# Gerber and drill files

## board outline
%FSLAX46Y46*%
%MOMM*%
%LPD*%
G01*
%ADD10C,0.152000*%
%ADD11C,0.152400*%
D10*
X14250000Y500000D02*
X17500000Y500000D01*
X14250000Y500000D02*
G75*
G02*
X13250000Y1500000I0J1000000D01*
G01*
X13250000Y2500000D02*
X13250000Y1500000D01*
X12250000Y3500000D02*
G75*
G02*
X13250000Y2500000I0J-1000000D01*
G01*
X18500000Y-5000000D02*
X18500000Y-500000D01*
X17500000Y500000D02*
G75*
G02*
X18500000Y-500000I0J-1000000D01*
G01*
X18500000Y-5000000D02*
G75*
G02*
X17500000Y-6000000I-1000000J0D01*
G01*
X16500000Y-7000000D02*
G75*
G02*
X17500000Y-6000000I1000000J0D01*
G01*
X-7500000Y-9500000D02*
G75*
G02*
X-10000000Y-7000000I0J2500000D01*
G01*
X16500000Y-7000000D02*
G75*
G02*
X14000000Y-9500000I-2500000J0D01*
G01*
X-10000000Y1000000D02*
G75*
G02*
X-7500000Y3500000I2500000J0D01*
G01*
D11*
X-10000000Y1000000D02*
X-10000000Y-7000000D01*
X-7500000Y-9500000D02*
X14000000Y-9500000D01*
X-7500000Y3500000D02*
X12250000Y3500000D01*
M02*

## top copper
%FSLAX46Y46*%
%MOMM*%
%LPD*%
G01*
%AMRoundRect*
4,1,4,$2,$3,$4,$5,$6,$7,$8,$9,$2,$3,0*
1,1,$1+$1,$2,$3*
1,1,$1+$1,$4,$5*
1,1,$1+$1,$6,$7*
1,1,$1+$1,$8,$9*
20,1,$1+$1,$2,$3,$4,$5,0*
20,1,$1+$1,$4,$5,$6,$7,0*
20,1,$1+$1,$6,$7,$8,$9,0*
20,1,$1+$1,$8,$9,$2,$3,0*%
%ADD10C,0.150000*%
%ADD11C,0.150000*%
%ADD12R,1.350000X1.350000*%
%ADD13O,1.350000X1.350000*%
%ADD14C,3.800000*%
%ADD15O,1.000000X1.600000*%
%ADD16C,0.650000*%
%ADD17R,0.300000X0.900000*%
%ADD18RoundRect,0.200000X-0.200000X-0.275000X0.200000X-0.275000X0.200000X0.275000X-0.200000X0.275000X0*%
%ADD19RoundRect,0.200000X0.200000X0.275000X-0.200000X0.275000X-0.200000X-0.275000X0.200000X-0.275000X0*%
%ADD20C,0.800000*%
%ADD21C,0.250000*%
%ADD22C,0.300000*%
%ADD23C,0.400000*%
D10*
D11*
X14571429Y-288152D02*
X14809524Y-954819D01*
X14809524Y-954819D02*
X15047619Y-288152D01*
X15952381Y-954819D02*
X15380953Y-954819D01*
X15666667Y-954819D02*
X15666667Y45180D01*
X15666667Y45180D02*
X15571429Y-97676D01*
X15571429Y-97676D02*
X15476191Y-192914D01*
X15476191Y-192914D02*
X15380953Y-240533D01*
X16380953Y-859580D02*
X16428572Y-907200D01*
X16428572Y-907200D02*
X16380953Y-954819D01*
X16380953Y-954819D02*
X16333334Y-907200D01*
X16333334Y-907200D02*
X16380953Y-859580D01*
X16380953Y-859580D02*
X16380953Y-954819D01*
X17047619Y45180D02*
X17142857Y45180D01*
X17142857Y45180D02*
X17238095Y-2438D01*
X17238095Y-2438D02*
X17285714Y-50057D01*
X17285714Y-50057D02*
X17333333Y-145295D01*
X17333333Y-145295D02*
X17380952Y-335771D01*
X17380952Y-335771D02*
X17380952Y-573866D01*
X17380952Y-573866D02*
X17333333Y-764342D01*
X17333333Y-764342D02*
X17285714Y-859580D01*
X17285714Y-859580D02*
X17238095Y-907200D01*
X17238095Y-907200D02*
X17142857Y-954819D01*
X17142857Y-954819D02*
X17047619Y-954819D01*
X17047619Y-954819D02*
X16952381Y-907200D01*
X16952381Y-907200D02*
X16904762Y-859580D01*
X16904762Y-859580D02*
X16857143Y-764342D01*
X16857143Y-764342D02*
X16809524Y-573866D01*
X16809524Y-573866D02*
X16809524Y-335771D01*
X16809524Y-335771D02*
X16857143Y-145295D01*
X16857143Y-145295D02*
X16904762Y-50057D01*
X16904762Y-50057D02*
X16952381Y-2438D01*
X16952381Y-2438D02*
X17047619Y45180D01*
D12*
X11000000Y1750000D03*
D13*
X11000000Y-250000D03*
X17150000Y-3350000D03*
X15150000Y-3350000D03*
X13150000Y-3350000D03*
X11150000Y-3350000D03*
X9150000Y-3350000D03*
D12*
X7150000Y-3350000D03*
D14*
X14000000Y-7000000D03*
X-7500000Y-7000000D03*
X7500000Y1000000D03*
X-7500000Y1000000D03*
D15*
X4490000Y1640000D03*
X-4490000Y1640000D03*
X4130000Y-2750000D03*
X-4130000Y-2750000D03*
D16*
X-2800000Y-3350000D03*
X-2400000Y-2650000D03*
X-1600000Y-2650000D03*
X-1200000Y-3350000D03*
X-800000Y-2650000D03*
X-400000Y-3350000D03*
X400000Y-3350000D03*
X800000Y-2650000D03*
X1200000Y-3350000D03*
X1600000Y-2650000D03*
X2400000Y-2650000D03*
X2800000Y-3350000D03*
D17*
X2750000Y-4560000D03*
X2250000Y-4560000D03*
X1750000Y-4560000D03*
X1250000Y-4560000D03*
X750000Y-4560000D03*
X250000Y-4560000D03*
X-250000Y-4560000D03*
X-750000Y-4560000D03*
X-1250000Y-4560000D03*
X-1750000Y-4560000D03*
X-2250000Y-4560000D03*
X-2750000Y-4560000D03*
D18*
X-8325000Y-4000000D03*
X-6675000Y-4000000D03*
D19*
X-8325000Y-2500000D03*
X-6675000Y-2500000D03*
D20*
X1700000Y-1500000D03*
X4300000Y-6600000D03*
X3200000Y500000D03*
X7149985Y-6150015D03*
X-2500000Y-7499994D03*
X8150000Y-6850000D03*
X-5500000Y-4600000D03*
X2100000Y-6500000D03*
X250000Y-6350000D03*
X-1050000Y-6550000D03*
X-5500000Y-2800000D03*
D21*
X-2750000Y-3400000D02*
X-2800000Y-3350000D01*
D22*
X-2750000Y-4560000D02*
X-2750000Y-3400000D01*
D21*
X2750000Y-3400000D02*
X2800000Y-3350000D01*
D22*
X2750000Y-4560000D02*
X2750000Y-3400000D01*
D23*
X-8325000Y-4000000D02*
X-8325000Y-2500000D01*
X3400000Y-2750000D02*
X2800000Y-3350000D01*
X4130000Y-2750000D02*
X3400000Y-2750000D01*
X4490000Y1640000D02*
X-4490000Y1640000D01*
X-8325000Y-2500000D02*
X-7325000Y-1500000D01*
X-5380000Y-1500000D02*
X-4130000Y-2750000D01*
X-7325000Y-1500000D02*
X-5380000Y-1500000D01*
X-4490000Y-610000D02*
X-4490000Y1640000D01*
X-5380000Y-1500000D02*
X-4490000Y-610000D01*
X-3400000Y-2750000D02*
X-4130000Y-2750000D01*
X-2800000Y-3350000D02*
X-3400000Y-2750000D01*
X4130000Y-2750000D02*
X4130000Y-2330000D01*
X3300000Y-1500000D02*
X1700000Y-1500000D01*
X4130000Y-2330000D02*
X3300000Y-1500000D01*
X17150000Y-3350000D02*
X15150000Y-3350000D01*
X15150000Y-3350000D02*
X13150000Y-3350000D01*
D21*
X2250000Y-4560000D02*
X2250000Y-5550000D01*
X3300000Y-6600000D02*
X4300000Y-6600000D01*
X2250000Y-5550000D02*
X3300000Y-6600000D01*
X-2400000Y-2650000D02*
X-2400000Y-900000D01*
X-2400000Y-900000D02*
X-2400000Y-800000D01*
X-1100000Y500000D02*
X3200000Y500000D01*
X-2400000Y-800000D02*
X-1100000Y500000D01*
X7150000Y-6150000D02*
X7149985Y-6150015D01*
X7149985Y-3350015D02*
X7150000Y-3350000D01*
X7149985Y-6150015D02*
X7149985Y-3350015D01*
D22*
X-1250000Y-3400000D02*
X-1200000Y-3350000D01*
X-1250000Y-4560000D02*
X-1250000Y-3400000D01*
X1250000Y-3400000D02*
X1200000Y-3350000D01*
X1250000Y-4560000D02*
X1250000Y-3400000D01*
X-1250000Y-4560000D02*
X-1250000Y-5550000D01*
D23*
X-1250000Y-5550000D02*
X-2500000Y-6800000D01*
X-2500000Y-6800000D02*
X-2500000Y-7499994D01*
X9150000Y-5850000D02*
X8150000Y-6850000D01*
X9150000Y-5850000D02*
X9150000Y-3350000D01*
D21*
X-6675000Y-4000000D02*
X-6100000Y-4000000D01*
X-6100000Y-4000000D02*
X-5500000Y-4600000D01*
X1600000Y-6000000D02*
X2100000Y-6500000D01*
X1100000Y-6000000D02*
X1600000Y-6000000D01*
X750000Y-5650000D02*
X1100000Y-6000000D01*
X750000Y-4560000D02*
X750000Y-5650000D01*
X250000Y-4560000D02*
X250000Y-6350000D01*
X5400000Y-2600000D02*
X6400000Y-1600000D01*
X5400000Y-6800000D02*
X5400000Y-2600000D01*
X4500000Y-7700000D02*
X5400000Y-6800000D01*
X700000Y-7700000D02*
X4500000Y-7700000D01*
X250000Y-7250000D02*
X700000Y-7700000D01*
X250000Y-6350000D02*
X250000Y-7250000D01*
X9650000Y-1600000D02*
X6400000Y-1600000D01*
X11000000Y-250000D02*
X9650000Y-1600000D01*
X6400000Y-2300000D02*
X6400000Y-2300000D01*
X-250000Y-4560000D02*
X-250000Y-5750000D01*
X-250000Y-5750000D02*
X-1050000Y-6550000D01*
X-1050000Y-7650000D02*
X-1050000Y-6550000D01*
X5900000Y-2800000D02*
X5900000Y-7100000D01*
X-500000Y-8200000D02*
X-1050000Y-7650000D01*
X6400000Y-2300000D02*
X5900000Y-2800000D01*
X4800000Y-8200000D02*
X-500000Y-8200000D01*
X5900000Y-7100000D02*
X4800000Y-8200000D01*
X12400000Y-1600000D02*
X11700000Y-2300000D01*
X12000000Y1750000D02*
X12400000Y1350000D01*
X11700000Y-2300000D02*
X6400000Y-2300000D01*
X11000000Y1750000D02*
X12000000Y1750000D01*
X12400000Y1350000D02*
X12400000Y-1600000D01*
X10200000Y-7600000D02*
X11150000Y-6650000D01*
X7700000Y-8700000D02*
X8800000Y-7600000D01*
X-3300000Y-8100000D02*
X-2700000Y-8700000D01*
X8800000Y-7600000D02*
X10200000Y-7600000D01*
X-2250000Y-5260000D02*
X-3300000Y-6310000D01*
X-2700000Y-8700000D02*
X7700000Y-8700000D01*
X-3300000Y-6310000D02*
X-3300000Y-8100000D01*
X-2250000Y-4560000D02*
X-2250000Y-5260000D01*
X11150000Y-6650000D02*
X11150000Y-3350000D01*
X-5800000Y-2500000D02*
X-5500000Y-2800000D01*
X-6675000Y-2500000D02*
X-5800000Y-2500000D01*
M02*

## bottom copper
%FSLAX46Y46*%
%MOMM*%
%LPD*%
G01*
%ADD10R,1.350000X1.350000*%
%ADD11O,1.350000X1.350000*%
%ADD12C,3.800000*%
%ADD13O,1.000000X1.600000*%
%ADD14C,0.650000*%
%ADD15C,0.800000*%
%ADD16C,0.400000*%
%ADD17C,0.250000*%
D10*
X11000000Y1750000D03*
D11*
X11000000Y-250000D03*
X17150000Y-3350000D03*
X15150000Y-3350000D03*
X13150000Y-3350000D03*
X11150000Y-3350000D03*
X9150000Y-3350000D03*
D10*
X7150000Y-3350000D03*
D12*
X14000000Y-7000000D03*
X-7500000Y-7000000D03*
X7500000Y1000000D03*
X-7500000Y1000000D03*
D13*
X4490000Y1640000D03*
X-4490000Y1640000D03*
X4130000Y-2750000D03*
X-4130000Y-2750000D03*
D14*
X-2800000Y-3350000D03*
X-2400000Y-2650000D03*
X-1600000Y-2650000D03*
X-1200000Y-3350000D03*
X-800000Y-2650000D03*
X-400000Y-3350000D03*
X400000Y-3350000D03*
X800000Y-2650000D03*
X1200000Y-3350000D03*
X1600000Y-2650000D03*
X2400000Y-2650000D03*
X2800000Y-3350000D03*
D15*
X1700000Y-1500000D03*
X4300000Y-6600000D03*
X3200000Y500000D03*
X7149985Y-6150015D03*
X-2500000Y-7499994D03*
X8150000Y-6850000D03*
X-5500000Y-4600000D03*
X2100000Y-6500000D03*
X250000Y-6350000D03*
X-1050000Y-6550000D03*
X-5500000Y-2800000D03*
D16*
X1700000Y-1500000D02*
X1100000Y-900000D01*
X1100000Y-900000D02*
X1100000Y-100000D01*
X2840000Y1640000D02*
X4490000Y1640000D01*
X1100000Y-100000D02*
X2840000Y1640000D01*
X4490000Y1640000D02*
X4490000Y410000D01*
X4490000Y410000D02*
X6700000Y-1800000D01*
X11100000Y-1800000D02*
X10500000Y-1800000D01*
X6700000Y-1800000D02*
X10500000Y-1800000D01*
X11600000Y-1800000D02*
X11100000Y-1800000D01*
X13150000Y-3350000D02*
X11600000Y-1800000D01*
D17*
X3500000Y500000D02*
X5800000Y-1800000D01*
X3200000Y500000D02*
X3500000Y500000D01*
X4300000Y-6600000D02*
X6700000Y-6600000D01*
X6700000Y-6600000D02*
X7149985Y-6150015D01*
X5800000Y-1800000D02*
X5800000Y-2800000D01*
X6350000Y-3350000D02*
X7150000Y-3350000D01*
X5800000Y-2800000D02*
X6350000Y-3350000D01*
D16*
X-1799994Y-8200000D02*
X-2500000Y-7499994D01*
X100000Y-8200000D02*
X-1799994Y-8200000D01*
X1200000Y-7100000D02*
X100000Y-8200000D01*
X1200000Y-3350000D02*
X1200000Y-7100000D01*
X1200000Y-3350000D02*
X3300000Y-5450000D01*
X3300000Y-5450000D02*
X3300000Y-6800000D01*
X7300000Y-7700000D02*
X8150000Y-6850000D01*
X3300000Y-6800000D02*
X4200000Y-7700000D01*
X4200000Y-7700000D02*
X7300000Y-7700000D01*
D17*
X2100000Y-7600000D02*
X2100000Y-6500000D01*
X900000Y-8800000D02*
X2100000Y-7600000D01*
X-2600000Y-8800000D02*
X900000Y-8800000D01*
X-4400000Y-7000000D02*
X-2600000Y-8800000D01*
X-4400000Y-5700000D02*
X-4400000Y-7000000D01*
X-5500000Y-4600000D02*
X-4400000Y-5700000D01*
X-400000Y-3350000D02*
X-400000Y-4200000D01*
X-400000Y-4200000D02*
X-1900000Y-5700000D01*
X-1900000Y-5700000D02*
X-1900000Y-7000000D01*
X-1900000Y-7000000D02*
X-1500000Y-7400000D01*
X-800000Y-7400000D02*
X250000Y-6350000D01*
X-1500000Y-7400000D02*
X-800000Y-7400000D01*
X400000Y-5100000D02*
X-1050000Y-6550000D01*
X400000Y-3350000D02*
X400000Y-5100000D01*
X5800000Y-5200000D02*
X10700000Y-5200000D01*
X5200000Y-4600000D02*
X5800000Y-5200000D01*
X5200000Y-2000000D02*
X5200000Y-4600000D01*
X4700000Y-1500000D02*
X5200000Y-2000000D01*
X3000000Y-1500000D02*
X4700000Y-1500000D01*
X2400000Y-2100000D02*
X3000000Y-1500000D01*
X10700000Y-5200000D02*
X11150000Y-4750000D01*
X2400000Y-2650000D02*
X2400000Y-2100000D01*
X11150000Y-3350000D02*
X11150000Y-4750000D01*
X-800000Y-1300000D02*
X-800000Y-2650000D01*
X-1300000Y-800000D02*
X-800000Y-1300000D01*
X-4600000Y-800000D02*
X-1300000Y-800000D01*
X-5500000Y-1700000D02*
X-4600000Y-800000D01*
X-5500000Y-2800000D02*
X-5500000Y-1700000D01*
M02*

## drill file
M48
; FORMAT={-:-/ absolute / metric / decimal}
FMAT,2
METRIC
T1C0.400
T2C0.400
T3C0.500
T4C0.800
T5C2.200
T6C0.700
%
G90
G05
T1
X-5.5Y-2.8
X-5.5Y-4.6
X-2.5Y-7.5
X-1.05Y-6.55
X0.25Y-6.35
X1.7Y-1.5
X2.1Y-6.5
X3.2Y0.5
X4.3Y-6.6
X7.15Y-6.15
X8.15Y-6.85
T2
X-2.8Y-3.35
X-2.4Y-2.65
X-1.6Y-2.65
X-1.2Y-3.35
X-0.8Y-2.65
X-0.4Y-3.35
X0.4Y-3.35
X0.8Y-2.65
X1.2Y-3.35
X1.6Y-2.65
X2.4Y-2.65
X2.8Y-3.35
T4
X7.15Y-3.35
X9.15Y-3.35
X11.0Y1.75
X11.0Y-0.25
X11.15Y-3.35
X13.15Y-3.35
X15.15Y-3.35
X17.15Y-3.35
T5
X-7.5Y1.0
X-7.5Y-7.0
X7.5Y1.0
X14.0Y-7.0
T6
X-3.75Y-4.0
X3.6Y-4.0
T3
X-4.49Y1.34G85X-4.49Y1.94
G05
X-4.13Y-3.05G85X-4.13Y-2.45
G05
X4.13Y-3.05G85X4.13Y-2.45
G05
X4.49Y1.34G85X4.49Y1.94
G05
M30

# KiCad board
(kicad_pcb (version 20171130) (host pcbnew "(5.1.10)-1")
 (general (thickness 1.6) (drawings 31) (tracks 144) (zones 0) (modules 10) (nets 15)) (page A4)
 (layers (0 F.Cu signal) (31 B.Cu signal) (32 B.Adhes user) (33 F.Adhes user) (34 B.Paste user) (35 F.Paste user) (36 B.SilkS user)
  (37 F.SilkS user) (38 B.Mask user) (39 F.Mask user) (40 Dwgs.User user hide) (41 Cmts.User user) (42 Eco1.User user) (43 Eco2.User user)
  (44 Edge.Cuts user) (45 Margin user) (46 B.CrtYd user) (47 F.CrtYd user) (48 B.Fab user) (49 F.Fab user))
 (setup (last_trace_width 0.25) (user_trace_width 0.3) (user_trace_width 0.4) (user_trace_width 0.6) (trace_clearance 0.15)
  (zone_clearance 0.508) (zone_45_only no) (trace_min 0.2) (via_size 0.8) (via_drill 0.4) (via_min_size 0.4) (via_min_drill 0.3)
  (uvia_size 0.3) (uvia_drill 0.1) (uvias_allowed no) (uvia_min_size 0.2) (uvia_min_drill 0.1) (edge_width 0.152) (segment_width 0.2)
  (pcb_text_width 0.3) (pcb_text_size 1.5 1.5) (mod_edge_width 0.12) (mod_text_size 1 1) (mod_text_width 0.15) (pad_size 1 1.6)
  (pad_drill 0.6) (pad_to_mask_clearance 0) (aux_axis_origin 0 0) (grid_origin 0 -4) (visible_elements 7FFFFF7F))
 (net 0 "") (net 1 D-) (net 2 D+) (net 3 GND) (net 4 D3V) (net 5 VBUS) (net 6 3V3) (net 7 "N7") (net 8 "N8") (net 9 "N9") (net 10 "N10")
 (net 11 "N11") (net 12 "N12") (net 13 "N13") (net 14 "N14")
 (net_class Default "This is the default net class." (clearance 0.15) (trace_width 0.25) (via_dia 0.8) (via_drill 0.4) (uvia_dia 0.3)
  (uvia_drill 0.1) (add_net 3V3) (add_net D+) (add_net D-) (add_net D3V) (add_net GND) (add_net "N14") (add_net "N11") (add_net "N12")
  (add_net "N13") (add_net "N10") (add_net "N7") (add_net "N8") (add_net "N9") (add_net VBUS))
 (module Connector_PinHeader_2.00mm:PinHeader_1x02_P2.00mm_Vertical (layer F.Cu) (at 11 -1.75)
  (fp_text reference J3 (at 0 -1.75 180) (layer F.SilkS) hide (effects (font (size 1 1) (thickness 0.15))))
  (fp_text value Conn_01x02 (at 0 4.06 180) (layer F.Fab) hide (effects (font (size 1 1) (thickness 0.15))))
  (pad 1 thru_hole rect (at 0 0) (size 1.35 1.35) (drill 0.8) (layers *.Cu *.Mask) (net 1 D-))
  (pad 2 thru_hole oval (at 0 2) (size 1.35 1.35) (drill 0.8) (layers *.Cu *.Mask) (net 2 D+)))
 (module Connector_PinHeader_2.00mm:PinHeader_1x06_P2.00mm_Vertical (layer F.Cu) (at 7.15 3.35 90)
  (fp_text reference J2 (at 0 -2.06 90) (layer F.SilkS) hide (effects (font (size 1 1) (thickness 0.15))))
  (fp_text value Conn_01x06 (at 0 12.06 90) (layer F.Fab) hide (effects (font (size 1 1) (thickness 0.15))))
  (pad 6 thru_hole oval (at 0 10 90) (size 1.35 1.35) (drill 0.8) (layers *.Cu *.Mask) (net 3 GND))
  (pad 5 thru_hole oval (at 0 8 90) (size 1.35 1.35) (drill 0.8) (layers *.Cu *.Mask) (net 3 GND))
  (pad 4 thru_hole oval (at 0 6 90) (size 1.35 1.35) (drill 0.8) (layers *.Cu *.Mask) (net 3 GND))
  (pad 3 thru_hole oval (at 0 4 90) (size 1.35 1.35) (drill 0.8) (layers *.Cu *.Mask) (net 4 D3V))
  (pad 2 thru_hole oval (at 0 2 90) (size 1.35 1.35) (drill 0.8) (layers *.Cu *.Mask) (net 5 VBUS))
  (pad 1 thru_hole rect (at 0 0 90) (size 1.35 1.35) (drill 0.8) (layers *.Cu *.Mask) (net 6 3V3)))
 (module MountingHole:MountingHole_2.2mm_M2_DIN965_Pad (layer F.Cu) (at 14 7)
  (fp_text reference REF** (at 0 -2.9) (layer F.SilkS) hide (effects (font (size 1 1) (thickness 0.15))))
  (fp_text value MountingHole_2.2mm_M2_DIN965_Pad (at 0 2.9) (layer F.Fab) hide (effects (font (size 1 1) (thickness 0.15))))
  (pad 1 thru_hole circle (at 0 0) (size 3.8 3.8) (drill 2.2) (layers *.Cu *.Mask)))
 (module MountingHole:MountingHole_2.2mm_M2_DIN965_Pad (layer F.Cu) (at -7.5 7)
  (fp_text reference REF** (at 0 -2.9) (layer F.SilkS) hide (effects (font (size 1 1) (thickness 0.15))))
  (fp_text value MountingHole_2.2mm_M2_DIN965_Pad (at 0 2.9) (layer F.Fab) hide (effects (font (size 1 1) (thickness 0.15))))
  (pad 1 thru_hole circle (at 0 0) (size 3.8 3.8) (drill 2.2) (layers *.Cu *.Mask)))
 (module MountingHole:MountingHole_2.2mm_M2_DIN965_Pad (layer F.Cu) (at 7.5 -1)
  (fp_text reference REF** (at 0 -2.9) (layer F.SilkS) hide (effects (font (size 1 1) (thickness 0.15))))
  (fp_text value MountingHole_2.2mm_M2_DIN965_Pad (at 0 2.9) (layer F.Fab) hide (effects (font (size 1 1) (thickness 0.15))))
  (pad 1 thru_hole circle (at 0 0) (size 3.8 3.8) (drill 2.2) (layers *.Cu *.Mask)))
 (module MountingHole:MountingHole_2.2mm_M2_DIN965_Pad (layer F.Cu) (at -7.5 -1)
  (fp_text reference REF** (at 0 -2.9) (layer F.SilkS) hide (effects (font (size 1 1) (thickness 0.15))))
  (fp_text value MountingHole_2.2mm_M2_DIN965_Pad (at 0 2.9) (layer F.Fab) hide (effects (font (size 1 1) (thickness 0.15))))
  (pad 1 thru_hole circle (at 0 0) (size 3.8 3.8) (drill 2.2) (layers *.Cu *.Mask)))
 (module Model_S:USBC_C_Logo (layer F.Cu) (at -3.5 7.5)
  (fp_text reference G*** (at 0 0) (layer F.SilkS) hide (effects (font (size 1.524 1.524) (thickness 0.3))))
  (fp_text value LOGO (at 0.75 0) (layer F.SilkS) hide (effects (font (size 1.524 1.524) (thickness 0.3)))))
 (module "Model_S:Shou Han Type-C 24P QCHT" (layer F.Cu) (at 0 -3.5 180)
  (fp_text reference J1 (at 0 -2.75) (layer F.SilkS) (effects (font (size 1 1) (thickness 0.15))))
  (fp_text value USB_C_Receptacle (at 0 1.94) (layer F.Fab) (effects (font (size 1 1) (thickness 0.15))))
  (pad S1 thru_hole oval (at -4.49 -1.86 180) (size 1 1.6) (drill oval 0.5 1.1) (layers *.Cu *.Mask) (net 3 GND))
  (pad S1 thru_hole oval (at 4.49 -1.86 180) (size 1 1.6) (drill oval 0.5 1.1) (layers *.Cu *.Mask) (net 3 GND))
  (pad S1 thru_hole oval (at -4.13 -6.25 180) (size 1 1.6) (drill oval 0.5 1.1) (layers *.Cu *.Mask) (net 3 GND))
  (pad S1 thru_hole oval (at 4.13 -6.25 180) (size 1 1.6) (drill oval 0.5 1.1) (layers *.Cu *.Mask) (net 3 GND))
  (pad B1 thru_hole circle (at 2.8 -6.85 180) (size 0.65 0.65) (drill 0.4) (layers *.Cu *.Mask) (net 3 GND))
  (pad B2 thru_hole circle (at 2.4 -6.15 180) (size 0.65 0.65) (drill 0.4) (layers *.Cu *.Mask) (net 6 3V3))
  (pad B3 thru_hole circle (at 1.6 -6.15 180) (size 0.65 0.65) (drill 0.4) (layers *.Cu *.Mask) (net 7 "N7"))
  (pad B4 thru_hole circle (at 1.2 -6.85 180) (size 0.65 0.65) (drill 0.4) (layers *.Cu *.Mask) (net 5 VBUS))
  (pad B5 thru_hole circle (at 0.8 -6.15 180) (size 0.65 0.65) (drill 0.4) (layers *.Cu *.Mask) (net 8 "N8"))
  (pad B6 thru_hole circle (at 0.4 -6.85 180) (size 0.65 0.65) (drill 0.4) (layers *.Cu *.Mask) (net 2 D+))
  (pad B7 thru_hole circle (at -0.4 -6.85 180) (size 0.65 0.65) (drill 0.4) (layers *.Cu *.Mask) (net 1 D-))
  (pad B8 thru_hole circle (at -0.8 -6.15 180) (size 0.65 0.65) (drill 0.4) (layers *.Cu *.Mask) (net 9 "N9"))
  (pad B9 thru_hole circle (at -1.2 -6.85 180) (size 0.65 0.65) (drill 0.4) (layers *.Cu *.Mask) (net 5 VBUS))
  (pad B10 thru_hole circle (at -1.6 -6.15 180) (size 0.65 0.65) (drill 0.4) (layers *.Cu *.Mask) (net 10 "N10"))
  (pad B11 thru_hole circle (at -2.4 -6.15 180) (size 0.65 0.65) (drill 0.4) (layers *.Cu *.Mask) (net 4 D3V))
  (pad B12 thru_hole circle (at -2.8 -6.85 180) (size 0.65 0.65) (drill 0.4) (layers *.Cu *.Mask) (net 3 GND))
  (pad "" np_thru_hole circle (at -3.6 -7.5 180) (size 0.7 0.7) (drill 0.7) (layers *.Cu *.Mask))
  (pad "" np_thru_hole circle (at 3.75 -7.5 180) (size 0.7 0.7) (drill 0.7) (layers *.Cu *.Mask))
  (pad A1 smd rect (at -2.75 -8.06 180) (size 0.3 0.9) (layers F.Cu F.Paste F.Mask) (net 3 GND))
  (pad A2 smd rect (at -2.25 -8.06 180) (size 0.3 0.9) (layers F.Cu F.Paste F.Mask) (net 6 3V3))
  (pad A3 smd rect (at -1.75 -8.06 180) (size 0.3 0.9) (layers F.Cu F.Paste F.Mask) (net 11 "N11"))
  (pad A4 smd rect (at -1.25 -8.06 180) (size 0.3 0.9) (layers F.Cu F.Paste F.Mask) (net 5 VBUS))
  (pad A5 smd rect (at -0.75 -8.06 180) (size 0.3 0.9) (layers F.Cu F.Paste F.Mask) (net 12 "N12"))
  (pad A6 smd rect (at -0.25 -8.06 180) (size 0.3 0.9) (layers F.Cu F.Paste F.Mask) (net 2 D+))
  (pad A7 smd rect (at 0.25 -8.06 180) (size 0.3 0.9) (layers F.Cu F.Paste F.Mask) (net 1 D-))
  (pad A8 smd rect (at 0.75 -8.06 180) (size 0.3 0.9) (layers F.Cu F.Paste F.Mask) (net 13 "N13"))
  (pad A9 smd rect (at 1.25 -8.06 180) (size 0.3 0.9) (layers F.Cu F.Paste F.Mask) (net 5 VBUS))
  (pad A10 smd rect (at 1.75 -8.06 180) (size 0.3 0.9) (layers F.Cu F.Paste F.Mask) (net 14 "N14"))
  (pad A11 smd rect (at 2.25 -8.06 180) (size 0.3 0.9) (layers F.Cu F.Paste F.Mask) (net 4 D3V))
  (pad A12 smd rect (at 2.75 -8.06 180) (size 0.3 0.9) (layers F.Cu F.Paste F.Mask) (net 3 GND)))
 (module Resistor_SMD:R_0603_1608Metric (layer F.Cu) (at -7.5 4)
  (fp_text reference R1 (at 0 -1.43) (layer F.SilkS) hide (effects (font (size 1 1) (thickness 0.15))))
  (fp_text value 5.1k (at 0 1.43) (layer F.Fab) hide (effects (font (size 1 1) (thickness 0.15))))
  (pad 1 smd roundrect (at -0.825 0) (size 0.8 0.95) (layers F.Cu F.Paste F.Mask) (roundrect_rratio 0.25) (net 3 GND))
  (pad 2 smd roundrect (at 0.825 0) (size 0.8 0.95) (layers F.Cu F.Paste F.Mask) (roundrect_rratio 0.25) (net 12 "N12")))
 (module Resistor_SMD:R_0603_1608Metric (layer F.Cu) (at -7.5 2.5 180)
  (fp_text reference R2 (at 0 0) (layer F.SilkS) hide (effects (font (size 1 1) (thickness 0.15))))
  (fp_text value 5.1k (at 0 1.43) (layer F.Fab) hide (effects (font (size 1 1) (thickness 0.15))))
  (pad 2 smd roundrect (at 0.825 0 180) (size 0.8 0.95) (layers F.Cu F.Paste F.Mask) (roundrect_rratio 0.25) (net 3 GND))
  (pad 1 smd roundrect (at -0.825 0 180) (size 0.8 0.95) (layers F.Cu F.Paste F.Mask) (roundrect_rratio 0.25) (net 8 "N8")))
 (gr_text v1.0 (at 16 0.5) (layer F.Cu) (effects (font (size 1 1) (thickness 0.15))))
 (gr_line (start 14.25 -0.5) (end 17.5 -0.5) (layer Edge.Cuts) (width 0.152))
 (gr_arc (start 14.25 -1.5) (end 13.25 -1.5) (angle -90) (layer Edge.Cuts) (width 0.152))
 (gr_line (start 13.25 -2.5) (end 13.25 -1.5) (layer Edge.Cuts) (width 0.152))
 (gr_arc (start 12.25 -2.5) (end 13.25 -2.5) (angle -90) (layer Edge.Cuts) (width 0.152))
 (gr_line (start 18.5 5) (end 18.5 0.5) (layer Edge.Cuts) (width 0.152))
 (gr_arc (start 17.5 0.5) (end 18.5 0.5) (angle -90) (layer Edge.Cuts) (width 0.152))
 (gr_arc (start 17.5 5) (end 17.5 6) (angle -90) (layer Edge.Cuts) (width 0.152))
 (gr_arc (start 17.5 7) (end 17.5 6) (angle -90) (layer Edge.Cuts) (width 0.152))
 (gr_arc (start -7.5 7) (end -10 7) (angle -90) (layer Edge.Cuts) (width 0.152))
 (gr_arc (start 14 7) (end 14 9.5) (angle -90) (layer Edge.Cuts) (width 0.152))
 (gr_arc (start -7.5 -1) (end -7.5 -3.5) (angle -90) (layer Edge.Cuts) (width 0.152))
 (gr_line (start -10 -1) (end -10 7) (layer Edge.Cuts) (width 0.1524))
 (gr_line (start -7.5 9.5) (end 14 9.5) (layer Edge.Cuts) (width 0.1524))
 (gr_line (start -7.5 -3.5) (end 12.25 -3.5) (layer Edge.Cuts) (width 0.1524))
 (segment (start -2.75 3.4) (end -2.8 3.35) (width 0.25) (layer F.Cu) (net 3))
 (segment (start -2.75 4.56) (end -2.75 3.4) (width 0.3) (layer F.Cu) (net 3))
 (segment (start 2.75 3.4) (end 2.8 3.35) (width 0.25) (layer F.Cu) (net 3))
 (segment (start 2.75 4.56) (end 2.75 3.4) (width 0.3) (layer F.Cu) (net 3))
 (segment (start -8.325 4) (end -8.325 2.5) (width 0.4) (layer F.Cu) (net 3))
 (segment (start 3.4 2.75) (end 2.8 3.35) (width 0.4) (layer F.Cu) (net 3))
 (segment (start 4.13 2.75) (end 3.4 2.75) (width 0.4) (layer F.Cu) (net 3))
 (segment (start 4.49 -1.64) (end -4.49 -1.64) (width 0.4) (layer F.Cu) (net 3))
 (segment (start -8.325 2.5) (end -7.325 1.5) (width 0.4) (layer F.Cu) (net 3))
 (segment (start -5.38 1.5) (end -4.13 2.75) (width 0.4) (layer F.Cu) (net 3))
 (segment (start -7.325 1.5) (end -5.38 1.5) (width 0.4) (layer F.Cu) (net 3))
 (segment (start -4.49 0.61) (end -4.49 -1.64) (width 0.4) (layer F.Cu) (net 3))
 (segment (start -5.38 1.5) (end -4.49 0.61) (width 0.4) (layer F.Cu) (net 3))
 (segment (start -3.4 2.75) (end -4.13 2.75) (width 0.4) (layer F.Cu) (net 3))
 (segment (start -2.8 3.35) (end -3.4 2.75) (width 0.4) (layer F.Cu) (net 3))
 (segment (start 4.13 2.75) (end 4.13 2.33) (width 0.4) (layer F.Cu) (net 3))
 (via (at 1.7 1.5) (size 0.8) (drill 0.4) (layers F.Cu B.Cu) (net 3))
 (segment (start 3.3 1.5) (end 1.7 1.5) (width 0.4) (layer F.Cu) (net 3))
 (segment (start 4.13 2.33) (end 3.3 1.5) (width 0.4) (layer F.Cu) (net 3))
 (segment (start 1.7 1.5) (end 1.1 0.9) (width 0.4) (layer B.Cu) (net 3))
 (segment (start 1.1 0.9) (end 1.1 0.1) (width 0.4) (layer B.Cu) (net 3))
 (segment (start 2.84 -1.64) (end 4.49 -1.64) (width 0.4) (layer B.Cu) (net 3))
 (segment (start 1.1 0.1) (end 2.84 -1.64) (width 0.4) (layer B.Cu) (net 3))
 (segment (start 4.49 -1.64) (end 4.49 -0.41) (width 0.4) (layer B.Cu) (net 3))
 (segment (start 4.49 -0.41) (end 6.7 1.8) (width 0.4) (layer B.Cu) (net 3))
 (segment (start 11.1 1.8) (end 10.5 1.8) (width 0.4) (layer B.Cu) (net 3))
 (segment (start 6.7 1.8) (end 10.5 1.8) (width 0.4) (layer B.Cu) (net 3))
 (segment (start 17.15 3.35) (end 15.15 3.35) (width 0.4) (layer F.Cu) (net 3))
 (segment (start 15.15 3.35) (end 13.15 3.35) (width 0.4) (layer F.Cu) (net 3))
 (segment (start 11.6 1.8) (end 11.1 1.8) (width 0.4) (layer B.Cu) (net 3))
 (segment (start 13.15 3.35) (end 11.6 1.8) (width 0.4) (layer B.Cu) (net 3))
 (segment (start 2.25 4.56) (end 2.25 5.55) (width 0.25) (layer F.Cu) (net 6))
 (via (at 4.3 6.6) (size 0.8) (drill 0.4) (layers F.Cu B.Cu) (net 6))
 (segment (start 3.3 6.6) (end 4.3 6.6) (width 0.25) (layer F.Cu) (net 6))
 (segment (start 2.25 5.55) (end 3.3 6.6) (width 0.25) (layer F.Cu) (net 6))
 (segment (start -2.4 2.65) (end -2.4 0.9) (width 0.25) (layer F.Cu) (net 6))
 (segment (start -2.4 0.9) (end -2.4 0.8) (width 0.25) (layer F.Cu) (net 6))
 (via (at 3.2 -0.5) (size 0.8) (drill 0.4) (layers F.Cu B.Cu) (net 6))
 (segment (start -1.1 -0.5) (end 3.2 -0.5) (width 0.25) (layer F.Cu) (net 6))
 (segment (start -2.4 0.8) (end -1.1 -0.5) (width 0.25) (layer F.Cu) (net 6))
 (segment (start 3.5 -0.5) (end 5.8 1.8) (width 0.25) (layer B.Cu) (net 6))
 (segment (start 3.2 -0.5) (end 3.5 -0.5) (width 0.25) (layer B.Cu) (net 6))
 (segment (start 4.3 6.6) (end 6.7 6.6) (width 0.25) (layer B.Cu) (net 6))
 (via (at 7.149985 6.150015) (size 0.8) (drill 0.4) (layers F.Cu B.Cu) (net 6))
 (segment (start 6.7 6.6) (end 7.149985 6.150015) (width 0.25) (layer B.Cu) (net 6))
 (segment (start 7.15 6.15) (end 7.149985 6.150015) (width 0.25) (layer F.Cu) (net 6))
 (segment (start 7.149985 3.350015) (end 7.15 3.35) (width 0.25) (layer F.Cu) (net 6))
 (segment (start 7.149985 6.150015) (end 7.149985 3.350015) (width 0.25) (layer F.Cu) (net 6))
 (segment (start 5.8 1.8) (end 5.8 2.8) (width 0.25) (layer B.Cu) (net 6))
 (segment (start 6.35 3.35) (end 7.15 3.35) (width 0.25) (layer B.Cu) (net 6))
 (segment (start 5.8 2.8) (end 6.35 3.35) (width 0.25) (layer B.Cu) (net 6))
 (segment (start -1.25 3.4) (end -1.2 3.35) (width 0.3) (layer F.Cu) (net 5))
 (segment (start -1.25 4.56) (end -1.25 3.4) (width 0.3) (layer F.Cu) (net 5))
 (segment (start 1.25 3.4) (end 1.2 3.35) (width 0.3) (layer F.Cu) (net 5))
 (segment (start 1.25 4.56) (end 1.25 3.4) (width 0.3) (layer F.Cu) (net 5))
 (segment (start -1.25 4.56) (end -1.25 5.55) (width 0.3) (layer F.Cu) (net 5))
 (via (at -2.5 7.499994) (size 0.8) (drill 0.4) (layers F.Cu B.Cu) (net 5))
 (segment (start -1.25 5.55) (end -2.5 6.8) (width 0.4) (layer F.Cu) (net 5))
 (segment (start -2.5 6.8) (end -2.5 7.499994) (width 0.4) (layer F.Cu) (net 5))
 (segment (start -1.799994 8.2) (end -2.5 7.499994) (width 0.4) (layer B.Cu) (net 5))
 (segment (start 0.1 8.2) (end -1.799994 8.2) (width 0.4) (layer B.Cu) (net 5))
 (segment (start 1.2 7.1) (end 0.1 8.2) (width 0.4) (layer B.Cu) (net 5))
 (segment (start 1.2 3.35) (end 1.2 7.1) (width 0.4) (layer B.Cu) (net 5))
 (via (at 8.15 6.85) (size 0.8) (drill 0.4) (layers F.Cu B.Cu) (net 5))
 (segment (start 9.15 5.85) (end 8.15 6.85) (width 0.4) (layer F.Cu) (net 5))
 (segment (start 1.2 3.35) (end 3.3 5.45) (width 0.4) (layer B.Cu) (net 5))
 (segment (start 3.3 5.45) (end 3.3 6.8) (width 0.4) (layer B.Cu) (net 5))
 (segment (start 7.3 7.7) (end 8.15 6.85) (width 0.4) (layer B.Cu) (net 5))
 (segment (start 3.3 6.8) (end 4.2 7.7) (width 0.4) (layer B.Cu) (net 5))
 (segment (start 4.2 7.7) (end 7.3 7.7) (width 0.4) (layer B.Cu) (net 5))
 (segment (start 9.15 5.85) (end 9.15 3.35) (width 0.4) (layer F.Cu) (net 5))
 (segment (start -6.675 4) (end -6.1 4) (width 0.25) (layer F.Cu) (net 12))
 (via (at -5.5 4.6) (size 0.8) (drill 0.4) (layers F.Cu B.Cu) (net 12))
 (segment (start -6.1 4) (end -5.5 4.6) (width 0.25) (layer F.Cu) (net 12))
 (via (at 2.1 6.5) (size 0.8) (drill 0.4) (layers F.Cu B.Cu) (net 12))
 (segment (start 1.6 6) (end 2.1 6.5) (width 0.25) (layer F.Cu) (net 12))
 (segment (start 1.1 6) (end 1.6 6) (width 0.25) (layer F.Cu) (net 12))
 (segment (start 0.75 5.65) (end 1.1 6) (width 0.25) (layer F.Cu) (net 12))
 (segment (start 0.75 4.56) (end 0.75 5.65) (width 0.25) (layer F.Cu) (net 12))
 (segment (start 2.1 7.6) (end 2.1 6.5) (width 0.25) (layer B.Cu) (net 12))
 (segment (start 0.9 8.8) (end 2.1 7.6) (width 0.25) (layer B.Cu) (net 12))
 (segment (start -2.6 8.8) (end 0.9 8.8) (width 0.25) (layer B.Cu) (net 12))
 (segment (start -4.4 7) (end -2.6 8.8) (width 0.25) (layer B.Cu) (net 12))
 (segment (start -4.4 5.7) (end -4.4 7) (width 0.25) (layer B.Cu) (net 12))
 (segment (start -5.5 4.6) (end -4.4 5.7) (width 0.25) (layer B.Cu) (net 12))
 (segment (start -0.4 3.35) (end -0.4 4.2) (width 0.25) (layer B.Cu) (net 2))
 (segment (start -0.4 4.2) (end -1.9 5.7) (width 0.25) (layer B.Cu) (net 2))
 (segment (start -1.9 5.7) (end -1.9 7) (width 0.25) (layer B.Cu) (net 2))
 (segment (start -1.9 7) (end -1.5 7.4) (width 0.25) (layer B.Cu) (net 2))
 (via (at 0.25 6.35) (size 0.8) (drill 0.4) (layers F.Cu B.Cu) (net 2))
 (segment (start -0.8 7.4) (end 0.25 6.35) (width 0.25) (layer B.Cu) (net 2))
 (segment (start -1.5 7.4) (end -0.8 7.4) (width 0.25) (layer B.Cu) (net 2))
 (segment (start 0.25 4.56) (end 0.25 6.35) (width 0.25) (layer F.Cu) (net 2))
 (segment (start 5.4 2.6) (end 6.4 1.6) (width 0.25) (layer F.Cu) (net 2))
 (segment (start 5.4 6.8) (end 5.4 2.6) (width 0.25) (layer F.Cu) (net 2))
 (segment (start 4.5 7.7) (end 5.4 6.8) (width 0.25) (layer F.Cu) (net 2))
 (segment (start 0.7 7.7) (end 4.5 7.7) (width 0.25) (layer F.Cu) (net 2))
 (segment (start 0.25 7.25) (end 0.7 7.7) (width 0.25) (layer F.Cu) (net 2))
 (segment (start 0.25 6.35) (end 0.25 7.25) (width 0.25) (layer F.Cu) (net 2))
 (segment (start 9.65 1.6) (end 6.4 1.6) (width 0.25) (layer F.Cu) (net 2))
 (segment (start 11 0.25) (end 9.65 1.6) (width 0.25) (layer F.Cu) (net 2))
 (segment (start 6.4 2.3) (end 6.4 2.3) (width 0.25) (layer F.Cu) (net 1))
 (segment (start 0.4 5.1) (end -1.05 6.55) (width 0.25) (layer B.Cu) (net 1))
 (segment (start 0.4 3.35) (end 0.4 5.1) (width 0.25) (layer B.Cu) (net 1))
 (segment (start -0.25 4.56) (end -0.25 5.75) (width 0.25) (layer F.Cu) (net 1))
 (segment (start -0.25 5.75) (end -1.05 6.55) (width 0.25) (layer F.Cu) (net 1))
 (via (at -1.05 6.55) (size 0.8) (drill 0.4) (layers F.Cu B.Cu) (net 1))
 (segment (start -1.05 7.65) (end -1.05 6.55) (width 0.25) (layer F.Cu) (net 1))
 (segment (start 5.9 2.8) (end 5.9 7.1) (width 0.25) (layer F.Cu) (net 1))
 (segment (start -0.5 8.2) (end -1.05 7.65) (width 0.25) (layer F.Cu) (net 1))
 (segment (start 6.4 2.3) (end 5.9 2.8) (width 0.25) (layer F.Cu) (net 1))
 (segment (start 4.8 8.2) (end -0.5 8.2) (width 0.25) (layer F.Cu) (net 1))
 (segment (start 5.9 7.1) (end 4.8 8.2) (width 0.25) (layer F.Cu) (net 1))
 (segment (start 12.4 1.6) (end 11.7 2.3) (width 0.25) (layer F.Cu) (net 1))
 (segment (start 12 -1.75) (end 12.4 -1.35) (width 0.25) (layer F.Cu) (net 1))
 (segment (start 11.7 2.3) (end 6.4 2.3) (width 0.25) (layer F.Cu) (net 1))
 (segment (start 11 -1.75) (end 12 -1.75) (width 0.25) (layer F.Cu) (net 1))
 (segment (start 12.4 -1.35) (end 12.4 1.6) (width 0.25) (layer F.Cu) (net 1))
 (segment (start 5.8 5.2) (end 10.7 5.2) (width 0.25) (layer B.Cu) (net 4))
 (segment (start 5.2 4.6) (end 5.8 5.2) (width 0.25) (layer B.Cu) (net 4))
 (segment (start 5.2 2) (end 5.2 4.6) (width 0.25) (layer B.Cu) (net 4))
 (segment (start 4.7 1.5) (end 5.2 2) (width 0.25) (layer B.Cu) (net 4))
 (segment (start 3 1.5) (end 4.7 1.5) (width 0.25) (layer B.Cu) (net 4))
 (segment (start 2.4 2.1) (end 3 1.5) (width 0.25) (layer B.Cu) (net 4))
 (segment (start 10.7 5.2) (end 11.15 4.75) (width 0.25) (layer B.Cu) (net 4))
 (segment (start 2.4 2.65) (end 2.4 2.1) (width 0.25) (layer B.Cu) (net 4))
 (segment (start 10.2 7.6) (end 11.15 6.65) (width 0.25) (layer F.Cu) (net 4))
 (segment (start 7.7 8.7) (end 8.8 7.6) (width 0.25) (layer F.Cu) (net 4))
 (segment (start -3.3 8.1) (end -2.7 8.7) (width 0.25) (layer F.Cu) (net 4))
 (segment (start 8.8 7.6) (end 10.2 7.6) (width 0.25) (layer F.Cu) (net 4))
 (segment (start -2.25 5.26) (end -3.3 6.31) (width 0.25) (layer F.Cu) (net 4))
 (segment (start -2.7 8.7) (end 7.7 8.7) (width 0.25) (layer F.Cu) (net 4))
 (segment (start -3.3 6.31) (end -3.3 8.1) (width 0.25) (layer F.Cu) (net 4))
 (segment (start -2.25 4.56) (end -2.25 5.26) (width 0.25) (layer F.Cu) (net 4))
 (segment (start 11.15 3.35) (end 11.15 4.75) (width 0.25) (layer B.Cu) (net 4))
 (segment (start 11.15 6.65) (end 11.15 3.35) (width 0.25) (layer F.Cu) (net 4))
 (via (at -5.5 2.8) (size 0.8) (drill 0.4) (layers F.Cu B.Cu) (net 8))
 (segment (start -5.8 2.5) (end -5.5 2.8) (width 0.25) (layer F.Cu) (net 8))
 (segment (start -6.675 2.5) (end -5.8 2.5) (width 0.25) (layer F.Cu) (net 8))
 (segment (start -0.8 1.3) (end -0.8 2.65) (width 0.25) (layer B.Cu) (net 8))
 (segment (start -1.3 0.8) (end -0.8 1.3) (width 0.25) (layer B.Cu) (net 8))
 (segment (start -4.6 0.8) (end -1.3 0.8) (width 0.25) (layer B.Cu) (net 8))
 (segment (start -5.5 1.7) (end -4.6 0.8) (width 0.25) (layer B.Cu) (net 8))
 (segment (start -5.5 2.8) (end -5.5 1.7) (width 0.25) (layer B.Cu) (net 8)))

